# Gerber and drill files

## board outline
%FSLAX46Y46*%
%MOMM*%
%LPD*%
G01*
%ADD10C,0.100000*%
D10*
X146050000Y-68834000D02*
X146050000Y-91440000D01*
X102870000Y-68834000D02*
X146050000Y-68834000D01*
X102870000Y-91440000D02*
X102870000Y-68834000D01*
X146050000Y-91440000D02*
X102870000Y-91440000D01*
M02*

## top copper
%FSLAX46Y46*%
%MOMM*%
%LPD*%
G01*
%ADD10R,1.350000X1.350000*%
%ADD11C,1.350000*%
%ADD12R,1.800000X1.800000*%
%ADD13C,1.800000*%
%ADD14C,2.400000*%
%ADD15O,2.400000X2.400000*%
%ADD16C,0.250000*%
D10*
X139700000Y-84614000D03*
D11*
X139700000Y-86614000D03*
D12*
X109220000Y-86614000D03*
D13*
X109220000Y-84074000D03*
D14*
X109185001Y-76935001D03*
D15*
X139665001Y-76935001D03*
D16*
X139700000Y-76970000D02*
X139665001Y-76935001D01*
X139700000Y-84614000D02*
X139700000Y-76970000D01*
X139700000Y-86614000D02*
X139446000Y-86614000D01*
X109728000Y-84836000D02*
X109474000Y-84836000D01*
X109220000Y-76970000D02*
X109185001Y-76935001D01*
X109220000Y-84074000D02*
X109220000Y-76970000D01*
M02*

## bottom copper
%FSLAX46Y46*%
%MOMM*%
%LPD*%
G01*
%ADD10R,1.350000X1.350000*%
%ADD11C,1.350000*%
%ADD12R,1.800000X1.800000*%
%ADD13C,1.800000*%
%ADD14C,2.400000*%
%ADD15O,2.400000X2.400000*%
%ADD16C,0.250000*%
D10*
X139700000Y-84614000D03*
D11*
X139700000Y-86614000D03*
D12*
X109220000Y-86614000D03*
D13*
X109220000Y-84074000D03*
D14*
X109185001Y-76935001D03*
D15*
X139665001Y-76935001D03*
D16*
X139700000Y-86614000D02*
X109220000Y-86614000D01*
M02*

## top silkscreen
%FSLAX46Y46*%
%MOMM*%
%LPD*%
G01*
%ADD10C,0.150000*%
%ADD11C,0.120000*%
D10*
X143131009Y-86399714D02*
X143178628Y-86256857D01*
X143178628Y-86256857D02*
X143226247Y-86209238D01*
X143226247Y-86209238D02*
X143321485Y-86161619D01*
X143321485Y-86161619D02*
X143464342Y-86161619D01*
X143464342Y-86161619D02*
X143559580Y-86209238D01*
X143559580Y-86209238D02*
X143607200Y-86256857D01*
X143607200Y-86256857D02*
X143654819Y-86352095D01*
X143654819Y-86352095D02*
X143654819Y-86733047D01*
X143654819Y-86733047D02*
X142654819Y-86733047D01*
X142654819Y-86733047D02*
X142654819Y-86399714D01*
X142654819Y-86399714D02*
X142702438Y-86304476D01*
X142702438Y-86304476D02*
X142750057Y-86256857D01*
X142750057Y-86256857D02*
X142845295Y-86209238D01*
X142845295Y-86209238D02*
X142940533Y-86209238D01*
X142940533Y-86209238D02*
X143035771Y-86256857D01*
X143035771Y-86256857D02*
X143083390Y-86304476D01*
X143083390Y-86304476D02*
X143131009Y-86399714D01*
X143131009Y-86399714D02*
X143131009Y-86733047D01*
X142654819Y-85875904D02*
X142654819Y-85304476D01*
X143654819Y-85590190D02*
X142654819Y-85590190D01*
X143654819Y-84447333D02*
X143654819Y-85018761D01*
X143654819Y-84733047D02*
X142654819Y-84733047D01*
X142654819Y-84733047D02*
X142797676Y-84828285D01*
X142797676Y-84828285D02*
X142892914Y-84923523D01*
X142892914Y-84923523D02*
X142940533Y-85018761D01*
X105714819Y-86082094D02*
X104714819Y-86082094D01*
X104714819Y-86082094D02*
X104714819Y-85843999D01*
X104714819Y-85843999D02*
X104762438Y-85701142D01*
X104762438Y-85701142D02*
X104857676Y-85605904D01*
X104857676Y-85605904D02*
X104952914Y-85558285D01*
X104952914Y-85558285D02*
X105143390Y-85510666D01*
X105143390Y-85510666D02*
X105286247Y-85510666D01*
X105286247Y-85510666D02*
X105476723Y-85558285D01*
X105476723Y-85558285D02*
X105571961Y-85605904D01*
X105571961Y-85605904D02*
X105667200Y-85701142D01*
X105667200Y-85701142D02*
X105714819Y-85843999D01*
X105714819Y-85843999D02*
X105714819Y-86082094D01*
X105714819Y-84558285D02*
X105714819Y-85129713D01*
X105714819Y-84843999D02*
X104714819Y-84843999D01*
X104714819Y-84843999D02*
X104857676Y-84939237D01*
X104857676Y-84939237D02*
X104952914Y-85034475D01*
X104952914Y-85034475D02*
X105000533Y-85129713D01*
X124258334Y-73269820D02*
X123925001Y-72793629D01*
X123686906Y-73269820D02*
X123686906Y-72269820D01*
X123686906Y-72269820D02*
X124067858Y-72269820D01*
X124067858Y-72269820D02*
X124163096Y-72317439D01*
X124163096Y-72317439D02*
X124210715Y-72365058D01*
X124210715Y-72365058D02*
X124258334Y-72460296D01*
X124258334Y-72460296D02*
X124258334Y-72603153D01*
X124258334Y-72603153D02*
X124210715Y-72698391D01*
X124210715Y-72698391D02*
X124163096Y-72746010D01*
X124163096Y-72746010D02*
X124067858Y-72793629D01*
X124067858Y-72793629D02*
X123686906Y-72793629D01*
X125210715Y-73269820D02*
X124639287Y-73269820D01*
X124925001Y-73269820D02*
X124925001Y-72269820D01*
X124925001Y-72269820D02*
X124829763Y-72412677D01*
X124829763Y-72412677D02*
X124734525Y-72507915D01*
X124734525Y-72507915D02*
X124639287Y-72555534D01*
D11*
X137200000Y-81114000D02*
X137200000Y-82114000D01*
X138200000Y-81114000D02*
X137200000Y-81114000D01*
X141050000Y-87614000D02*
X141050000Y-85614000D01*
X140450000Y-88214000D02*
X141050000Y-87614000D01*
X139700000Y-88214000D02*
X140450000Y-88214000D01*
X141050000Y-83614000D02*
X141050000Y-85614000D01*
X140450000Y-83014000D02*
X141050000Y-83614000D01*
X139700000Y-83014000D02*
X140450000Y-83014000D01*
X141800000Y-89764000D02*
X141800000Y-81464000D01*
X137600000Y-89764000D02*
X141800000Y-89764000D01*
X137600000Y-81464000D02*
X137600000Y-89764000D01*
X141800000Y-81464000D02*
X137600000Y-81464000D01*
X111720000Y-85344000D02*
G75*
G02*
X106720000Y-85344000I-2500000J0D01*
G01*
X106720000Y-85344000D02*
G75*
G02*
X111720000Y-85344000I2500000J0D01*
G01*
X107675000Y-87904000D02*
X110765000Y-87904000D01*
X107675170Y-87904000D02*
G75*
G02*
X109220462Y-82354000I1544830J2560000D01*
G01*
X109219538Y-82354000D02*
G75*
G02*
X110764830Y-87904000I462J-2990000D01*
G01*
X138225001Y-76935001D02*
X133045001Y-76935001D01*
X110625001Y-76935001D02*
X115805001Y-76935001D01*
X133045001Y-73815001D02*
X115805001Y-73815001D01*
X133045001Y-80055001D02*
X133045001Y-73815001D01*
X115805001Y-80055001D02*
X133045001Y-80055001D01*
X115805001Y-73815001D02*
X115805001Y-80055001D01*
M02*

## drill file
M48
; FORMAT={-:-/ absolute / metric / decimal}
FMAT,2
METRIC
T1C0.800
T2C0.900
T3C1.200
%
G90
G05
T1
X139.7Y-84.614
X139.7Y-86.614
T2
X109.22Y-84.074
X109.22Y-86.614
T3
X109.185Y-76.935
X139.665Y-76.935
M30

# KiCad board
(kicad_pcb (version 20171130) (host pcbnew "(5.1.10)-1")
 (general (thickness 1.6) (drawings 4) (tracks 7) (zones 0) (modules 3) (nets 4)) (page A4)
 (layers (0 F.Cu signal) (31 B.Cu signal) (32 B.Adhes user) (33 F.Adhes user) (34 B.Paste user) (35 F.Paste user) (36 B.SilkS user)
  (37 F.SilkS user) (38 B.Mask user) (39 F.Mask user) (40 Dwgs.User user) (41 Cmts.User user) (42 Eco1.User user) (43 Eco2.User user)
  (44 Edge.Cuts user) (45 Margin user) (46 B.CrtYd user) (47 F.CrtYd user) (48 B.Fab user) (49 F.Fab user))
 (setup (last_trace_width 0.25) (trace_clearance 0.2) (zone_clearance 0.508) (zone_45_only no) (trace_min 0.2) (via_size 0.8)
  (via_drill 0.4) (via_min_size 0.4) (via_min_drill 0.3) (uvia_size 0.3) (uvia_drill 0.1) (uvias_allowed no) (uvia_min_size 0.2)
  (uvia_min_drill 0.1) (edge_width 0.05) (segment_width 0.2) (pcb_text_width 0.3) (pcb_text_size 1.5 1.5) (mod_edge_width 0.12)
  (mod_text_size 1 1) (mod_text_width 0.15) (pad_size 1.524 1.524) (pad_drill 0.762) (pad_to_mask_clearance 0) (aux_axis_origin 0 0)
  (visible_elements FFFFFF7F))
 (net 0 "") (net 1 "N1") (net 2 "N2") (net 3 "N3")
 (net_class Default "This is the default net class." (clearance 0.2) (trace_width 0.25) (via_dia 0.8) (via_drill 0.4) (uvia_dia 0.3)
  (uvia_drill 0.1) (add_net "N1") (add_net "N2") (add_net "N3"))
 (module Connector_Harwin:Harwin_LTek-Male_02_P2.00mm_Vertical (layer F.Cu) (at 139.7 84.614 270)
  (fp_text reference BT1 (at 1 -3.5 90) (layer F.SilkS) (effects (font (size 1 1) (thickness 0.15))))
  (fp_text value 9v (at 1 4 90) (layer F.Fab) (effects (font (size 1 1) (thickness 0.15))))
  (fp_line (start -3.5 2.5) (end -2.5 2.5) (layer F.SilkS) (width 0.12))
  (fp_line (start -3.5 1.5) (end -3.5 2.5) (layer F.SilkS) (width 0.12))
  (fp_line (start 3 -1.35) (end 1 -1.35) (layer F.SilkS) (width 0.12))
  (fp_line (start 3.6 -0.75) (end 3 -1.35) (layer F.SilkS) (width 0.12))
  (fp_line (start 3.6 0) (end 3.6 -0.75) (layer F.SilkS) (width 0.12))
  (fp_line (start -1 -1.35) (end 1 -1.35) (layer F.SilkS) (width 0.12))
  (fp_line (start -1.6 -0.75) (end -1 -1.35) (layer F.SilkS) (width 0.12))
  (fp_line (start -1.6 0) (end -1.6 -0.75) (layer F.SilkS) (width 0.12))
  (fp_line (start 5.15 -2.1) (end -3.15 -2.1) (layer F.SilkS) (width 0.12))
  (fp_line (start 5.15 2.1) (end 5.15 -2.1) (layer F.SilkS) (width 0.12))
  (fp_line (start -3.15 2.1) (end 5.15 2.1) (layer F.SilkS) (width 0.12))
  (fp_line (start -3.15 -2.1) (end -3.15 2.1) (layer F.SilkS) (width 0.12))
  (pad 1 thru_hole rect (at 0 0 270) (size 1.35 1.35) (drill 0.8) (layers *.Cu *.Mask) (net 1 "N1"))
  (pad 2 thru_hole circle (at 2 0 270) (size 1.35 1.35) (drill 0.8) (layers *.Cu *.Mask) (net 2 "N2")))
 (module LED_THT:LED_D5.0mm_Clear (layer F.Cu) (at 109.22 86.614 90)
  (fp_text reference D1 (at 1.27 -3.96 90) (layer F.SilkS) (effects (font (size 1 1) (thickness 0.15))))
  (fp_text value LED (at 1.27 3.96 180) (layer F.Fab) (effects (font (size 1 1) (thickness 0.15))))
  (fp_circle (center 1.27 0) (end 3.77 0) (layer F.SilkS) (width 0.12))
  (fp_line (start -1.29 -1.545) (end -1.29 1.545) (layer F.SilkS) (width 0.12))
  (fp_arc (start 1.27 0) (end -1.29 -1.54483) (angle 148.9) (layer F.SilkS) (width 0.12))
  (fp_arc (start 1.27 0) (end -1.29 1.54483) (angle -148.9) (layer F.SilkS) (width 0.12))
  (pad 1 thru_hole rect (at 0 0 90) (size 1.8 1.8) (drill 0.9) (layers *.Cu *.Mask) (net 2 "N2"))
  (pad 2 thru_hole circle (at 2.54 0 90) (size 1.8 1.8) (drill 0.9) (layers *.Cu *.Mask) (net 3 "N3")))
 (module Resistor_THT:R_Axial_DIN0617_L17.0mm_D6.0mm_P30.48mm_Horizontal (layer F.Cu) (at 109.185001 76.935001)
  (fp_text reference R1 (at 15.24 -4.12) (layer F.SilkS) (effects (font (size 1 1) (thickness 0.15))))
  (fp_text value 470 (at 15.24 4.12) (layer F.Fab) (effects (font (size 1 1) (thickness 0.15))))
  (fp_line (start 29.04 0) (end 23.86 0) (layer F.SilkS) (width 0.12))
  (fp_line (start 1.44 0) (end 6.62 0) (layer F.SilkS) (width 0.12))
  (fp_line (start 23.86 -3.12) (end 6.62 -3.12) (layer F.SilkS) (width 0.12))
  (fp_line (start 23.86 3.12) (end 23.86 -3.12) (layer F.SilkS) (width 0.12))
  (fp_line (start 6.62 3.12) (end 23.86 3.12) (layer F.SilkS) (width 0.12))
  (fp_line (start 6.62 -3.12) (end 6.62 3.12) (layer F.SilkS) (width 0.12))
  (pad 1 thru_hole circle (at 0 0) (size 2.4 2.4) (drill 1.2) (layers *.Cu *.Mask) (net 3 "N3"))
  (pad 2 thru_hole oval (at 30.48 0) (size 2.4 2.4) (drill 1.2) (layers *.Cu *.Mask) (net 1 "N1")))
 (gr_line (start 146.05 68.834) (end 146.05 91.44) (layer Edge.Cuts) (width 0.1))
 (gr_line (start 102.87 68.834) (end 146.05 68.834) (layer Edge.Cuts) (width 0.1))
 (gr_line (start 102.87 91.44) (end 102.87 68.834) (layer Edge.Cuts) (width 0.1))
 (gr_line (start 146.05 91.44) (end 102.87 91.44) (layer Edge.Cuts) (width 0.1))
 (segment (start 139.7 76.97) (end 139.665001 76.935001) (width 0.25) (layer F.Cu) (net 1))
 (segment (start 139.7 84.614) (end 139.7 76.97) (width 0.25) (layer F.Cu) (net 1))
 (segment (start 139.7 86.614) (end 139.446 86.614) (width 0.25) (layer F.Cu) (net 2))
 (segment (start 139.7 86.614) (end 109.22 86.614) (width 0.25) (layer B.Cu) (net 2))
 (segment (start 109.728 84.836) (end 109.474 84.836) (width 0.25) (layer F.Cu) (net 3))
 (segment (start 109.22 76.97) (end 109.185001 76.935001) (width 0.25) (layer F.Cu) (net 3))
 (segment (start 109.22 84.074) (end 109.22 76.97) (width 0.25) (layer F.Cu) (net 3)))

